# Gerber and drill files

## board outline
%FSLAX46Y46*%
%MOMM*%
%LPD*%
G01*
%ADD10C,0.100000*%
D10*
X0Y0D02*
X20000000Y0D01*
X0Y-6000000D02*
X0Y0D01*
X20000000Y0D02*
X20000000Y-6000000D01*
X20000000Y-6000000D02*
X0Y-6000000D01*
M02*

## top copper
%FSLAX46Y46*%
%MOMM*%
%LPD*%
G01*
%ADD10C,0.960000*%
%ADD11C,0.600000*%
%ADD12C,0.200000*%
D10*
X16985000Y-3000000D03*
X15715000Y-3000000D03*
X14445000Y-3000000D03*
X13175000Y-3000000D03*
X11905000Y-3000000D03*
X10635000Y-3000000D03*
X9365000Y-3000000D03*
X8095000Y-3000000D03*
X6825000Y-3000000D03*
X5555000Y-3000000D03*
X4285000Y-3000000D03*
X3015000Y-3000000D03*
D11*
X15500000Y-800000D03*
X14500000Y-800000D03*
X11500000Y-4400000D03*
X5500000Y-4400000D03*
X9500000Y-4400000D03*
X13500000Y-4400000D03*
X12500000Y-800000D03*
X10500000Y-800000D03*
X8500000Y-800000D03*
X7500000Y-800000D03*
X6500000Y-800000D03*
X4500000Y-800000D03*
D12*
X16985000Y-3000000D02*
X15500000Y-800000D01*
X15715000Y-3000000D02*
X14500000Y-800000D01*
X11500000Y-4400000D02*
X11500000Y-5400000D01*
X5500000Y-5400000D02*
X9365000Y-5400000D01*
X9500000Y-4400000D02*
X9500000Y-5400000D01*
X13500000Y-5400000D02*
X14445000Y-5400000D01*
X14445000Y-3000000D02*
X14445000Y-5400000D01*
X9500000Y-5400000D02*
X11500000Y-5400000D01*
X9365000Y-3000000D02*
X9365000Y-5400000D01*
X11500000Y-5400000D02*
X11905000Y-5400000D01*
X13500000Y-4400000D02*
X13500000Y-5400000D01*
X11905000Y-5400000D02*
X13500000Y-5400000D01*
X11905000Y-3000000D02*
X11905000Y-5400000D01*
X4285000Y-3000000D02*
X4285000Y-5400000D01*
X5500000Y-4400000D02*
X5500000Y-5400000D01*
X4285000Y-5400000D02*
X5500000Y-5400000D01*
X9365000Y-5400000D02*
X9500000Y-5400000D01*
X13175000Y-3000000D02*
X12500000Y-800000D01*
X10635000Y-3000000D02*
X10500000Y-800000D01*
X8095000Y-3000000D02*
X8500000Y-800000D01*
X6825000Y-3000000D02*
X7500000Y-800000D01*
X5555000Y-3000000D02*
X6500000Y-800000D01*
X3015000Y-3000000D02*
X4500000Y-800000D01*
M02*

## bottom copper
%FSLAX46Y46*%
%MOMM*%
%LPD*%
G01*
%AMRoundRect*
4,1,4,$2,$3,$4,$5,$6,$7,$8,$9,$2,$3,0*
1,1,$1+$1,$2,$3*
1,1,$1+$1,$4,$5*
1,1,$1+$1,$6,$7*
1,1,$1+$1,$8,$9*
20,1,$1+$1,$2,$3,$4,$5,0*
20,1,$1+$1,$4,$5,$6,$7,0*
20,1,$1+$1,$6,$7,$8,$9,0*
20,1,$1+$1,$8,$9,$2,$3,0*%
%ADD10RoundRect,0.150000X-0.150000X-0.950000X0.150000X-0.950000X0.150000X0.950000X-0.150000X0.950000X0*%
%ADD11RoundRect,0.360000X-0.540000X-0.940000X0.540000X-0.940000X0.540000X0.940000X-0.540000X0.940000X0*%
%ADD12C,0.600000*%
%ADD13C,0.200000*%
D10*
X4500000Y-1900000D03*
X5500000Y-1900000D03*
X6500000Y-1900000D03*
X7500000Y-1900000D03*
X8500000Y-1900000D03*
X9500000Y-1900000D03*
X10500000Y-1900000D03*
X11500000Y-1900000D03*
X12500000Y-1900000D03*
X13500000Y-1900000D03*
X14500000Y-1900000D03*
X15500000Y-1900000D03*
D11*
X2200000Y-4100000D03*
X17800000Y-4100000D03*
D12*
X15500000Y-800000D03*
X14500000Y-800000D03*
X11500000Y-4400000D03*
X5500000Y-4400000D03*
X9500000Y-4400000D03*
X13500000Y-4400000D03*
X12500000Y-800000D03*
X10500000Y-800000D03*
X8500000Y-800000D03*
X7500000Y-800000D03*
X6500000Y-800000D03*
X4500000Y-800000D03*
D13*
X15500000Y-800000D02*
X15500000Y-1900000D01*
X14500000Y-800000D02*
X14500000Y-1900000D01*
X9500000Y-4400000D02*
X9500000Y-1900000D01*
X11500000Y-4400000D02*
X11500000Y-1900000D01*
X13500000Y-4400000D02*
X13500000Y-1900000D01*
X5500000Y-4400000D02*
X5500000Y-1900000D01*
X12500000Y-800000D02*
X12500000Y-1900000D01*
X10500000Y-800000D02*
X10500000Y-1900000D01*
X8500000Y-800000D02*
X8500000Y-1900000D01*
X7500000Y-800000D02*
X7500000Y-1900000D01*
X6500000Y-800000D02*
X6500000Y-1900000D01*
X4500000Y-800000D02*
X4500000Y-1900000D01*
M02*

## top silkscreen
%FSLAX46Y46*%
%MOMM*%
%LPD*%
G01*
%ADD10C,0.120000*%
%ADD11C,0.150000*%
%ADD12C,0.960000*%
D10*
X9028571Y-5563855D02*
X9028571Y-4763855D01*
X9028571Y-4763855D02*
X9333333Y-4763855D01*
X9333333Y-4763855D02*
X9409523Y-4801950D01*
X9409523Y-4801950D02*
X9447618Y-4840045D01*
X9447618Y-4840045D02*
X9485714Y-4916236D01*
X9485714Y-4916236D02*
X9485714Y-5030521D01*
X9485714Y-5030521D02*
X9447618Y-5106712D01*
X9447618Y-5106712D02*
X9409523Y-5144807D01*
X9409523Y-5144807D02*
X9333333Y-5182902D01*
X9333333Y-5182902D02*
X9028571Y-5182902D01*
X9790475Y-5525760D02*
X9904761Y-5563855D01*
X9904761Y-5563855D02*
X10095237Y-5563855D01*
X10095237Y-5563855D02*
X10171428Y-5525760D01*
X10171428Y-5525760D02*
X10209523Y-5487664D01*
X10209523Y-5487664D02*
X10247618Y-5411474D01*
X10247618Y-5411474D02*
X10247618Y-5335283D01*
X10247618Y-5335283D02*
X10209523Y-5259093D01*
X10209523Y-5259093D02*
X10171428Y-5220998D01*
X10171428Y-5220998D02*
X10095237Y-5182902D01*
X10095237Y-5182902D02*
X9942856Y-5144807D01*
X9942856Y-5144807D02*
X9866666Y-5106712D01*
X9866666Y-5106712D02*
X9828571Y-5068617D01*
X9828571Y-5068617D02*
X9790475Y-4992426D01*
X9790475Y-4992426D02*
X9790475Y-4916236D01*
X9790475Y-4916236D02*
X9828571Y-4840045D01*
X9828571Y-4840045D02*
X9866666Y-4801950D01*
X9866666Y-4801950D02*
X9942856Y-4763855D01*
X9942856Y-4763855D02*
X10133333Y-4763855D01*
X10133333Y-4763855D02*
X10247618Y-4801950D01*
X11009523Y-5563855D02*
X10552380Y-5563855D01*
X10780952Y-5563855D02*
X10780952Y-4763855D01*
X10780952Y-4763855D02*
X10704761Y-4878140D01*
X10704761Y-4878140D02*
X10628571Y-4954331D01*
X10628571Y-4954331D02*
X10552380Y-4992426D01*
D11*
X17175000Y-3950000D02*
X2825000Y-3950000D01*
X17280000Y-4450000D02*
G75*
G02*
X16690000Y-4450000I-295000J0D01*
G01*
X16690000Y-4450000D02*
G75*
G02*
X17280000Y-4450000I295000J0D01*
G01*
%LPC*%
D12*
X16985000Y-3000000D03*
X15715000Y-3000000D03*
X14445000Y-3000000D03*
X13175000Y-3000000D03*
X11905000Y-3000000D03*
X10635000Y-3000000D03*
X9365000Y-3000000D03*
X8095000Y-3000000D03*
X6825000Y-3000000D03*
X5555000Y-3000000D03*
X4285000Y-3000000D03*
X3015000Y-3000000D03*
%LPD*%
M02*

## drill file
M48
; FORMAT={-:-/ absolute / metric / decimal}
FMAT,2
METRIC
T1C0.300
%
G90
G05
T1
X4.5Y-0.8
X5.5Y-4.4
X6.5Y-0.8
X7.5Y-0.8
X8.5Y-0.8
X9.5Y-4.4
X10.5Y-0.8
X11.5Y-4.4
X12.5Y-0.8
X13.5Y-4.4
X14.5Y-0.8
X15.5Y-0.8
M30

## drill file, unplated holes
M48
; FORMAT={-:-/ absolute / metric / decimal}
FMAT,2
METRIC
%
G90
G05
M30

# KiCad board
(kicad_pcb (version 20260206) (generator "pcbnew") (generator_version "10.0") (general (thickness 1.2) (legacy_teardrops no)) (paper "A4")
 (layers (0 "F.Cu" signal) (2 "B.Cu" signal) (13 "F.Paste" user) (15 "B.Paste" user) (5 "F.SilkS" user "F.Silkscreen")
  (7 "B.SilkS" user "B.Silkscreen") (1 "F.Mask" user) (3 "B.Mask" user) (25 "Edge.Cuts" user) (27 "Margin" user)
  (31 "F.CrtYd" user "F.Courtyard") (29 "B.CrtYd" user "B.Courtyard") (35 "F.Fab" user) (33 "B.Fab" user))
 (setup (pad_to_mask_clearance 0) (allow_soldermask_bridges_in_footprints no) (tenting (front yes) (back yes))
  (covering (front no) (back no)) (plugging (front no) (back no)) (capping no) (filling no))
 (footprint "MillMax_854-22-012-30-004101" (layer "F.Cu") (at 10 3 180)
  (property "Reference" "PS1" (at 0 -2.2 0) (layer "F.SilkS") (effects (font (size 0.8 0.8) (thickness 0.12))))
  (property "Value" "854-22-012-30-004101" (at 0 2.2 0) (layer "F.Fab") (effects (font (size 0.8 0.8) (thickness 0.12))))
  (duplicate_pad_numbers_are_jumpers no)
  (fp_line (start -7.175 -0.95) (end 7.175 -0.95) (stroke (width 0.15) (type solid)) (layer "F.SilkS"))
  (fp_circle (center -6.985 -1.45) (end -6.69 -1.45) (stroke (width 0.15) (type solid)) (fill no) (layer "F.SilkS"))
  (pad "1" smd circle (at -6.985 0) (size 0.96 0.96) (layers "F.Cu" "F.Mask" "F.Paste") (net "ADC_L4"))
  (pad "2" smd circle (at -5.715 0) (size 0.96 0.96) (layers "F.Cu" "F.Mask" "F.Paste") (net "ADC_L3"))
  (pad "3" smd circle (at -4.445 0) (size 0.96 0.96) (layers "F.Cu" "F.Mask" "F.Paste") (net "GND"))
  (pad "4" smd circle (at -3.175 0) (size 0.96 0.96) (layers "F.Cu" "F.Mask" "F.Paste") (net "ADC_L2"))
  (pad "5" smd circle (at -1.905 0) (size 0.96 0.96) (layers "F.Cu" "F.Mask" "F.Paste") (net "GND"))
  (pad "6" smd circle (at -0.635 0) (size 0.96 0.96) (layers "F.Cu" "F.Mask" "F.Paste") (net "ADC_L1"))
  (pad "7" smd circle (at 0.635 0) (size 0.96 0.96) (layers "F.Cu" "F.Mask" "F.Paste") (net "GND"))
  (pad "8" smd circle (at 1.905 0) (size 0.96 0.96) (layers "F.Cu" "F.Mask" "F.Paste") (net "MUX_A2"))
  (pad "9" smd circle (at 3.175 0) (size 0.96 0.96) (layers "F.Cu" "F.Mask" "F.Paste") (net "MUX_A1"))
  (pad "10" smd circle (at 4.445 0) (size 0.96 0.96) (layers "F.Cu" "F.Mask" "F.Paste") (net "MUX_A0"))
  (pad "11" smd circle (at 5.715 0) (size 0.96 0.96) (layers "F.Cu" "F.Mask" "F.Paste") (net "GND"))
  (pad "12" smd circle (at 6.985 0) (size 0.96 0.96) (layers "F.Cu" "F.Mask" "F.Paste") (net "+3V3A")))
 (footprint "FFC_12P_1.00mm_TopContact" (layer "B.Cu") (at 10 3)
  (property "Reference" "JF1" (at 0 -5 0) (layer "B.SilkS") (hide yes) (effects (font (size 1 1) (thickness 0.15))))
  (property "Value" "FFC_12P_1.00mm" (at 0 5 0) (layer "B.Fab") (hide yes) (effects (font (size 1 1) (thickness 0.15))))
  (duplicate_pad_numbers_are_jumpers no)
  (pad "1" smd roundrect (at -5.5 -1.1) (size 0.6 2.2) (layers "B.Cu" "B.Mask" "B.Paste") (roundrect_rratio 0.25) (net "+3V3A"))
  (pad "2" smd roundrect (at -4.5 -1.1) (size 0.6 2.2) (layers "B.Cu" "B.Mask" "B.Paste") (roundrect_rratio 0.25) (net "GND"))
  (pad "3" smd roundrect (at -3.5 -1.1) (size 0.6 2.2) (layers "B.Cu" "B.Mask" "B.Paste") (roundrect_rratio 0.25) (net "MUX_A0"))
  (pad "4" smd roundrect (at -2.5 -1.1) (size 0.6 2.2) (layers "B.Cu" "B.Mask" "B.Paste") (roundrect_rratio 0.25) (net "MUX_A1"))
  (pad "5" smd roundrect (at -1.5 -1.1) (size 0.6 2.2) (layers "B.Cu" "B.Mask" "B.Paste") (roundrect_rratio 0.25) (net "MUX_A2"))
  (pad "6" smd roundrect (at -0.5 -1.1) (size 0.6 2.2) (layers "B.Cu" "B.Mask" "B.Paste") (roundrect_rratio 0.25) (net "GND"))
  (pad "7" smd roundrect (at 0.5 -1.1) (size 0.6 2.2) (layers "B.Cu" "B.Mask" "B.Paste") (roundrect_rratio 0.25) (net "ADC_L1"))
  (pad "8" smd roundrect (at 1.5 -1.1) (size 0.6 2.2) (layers "B.Cu" "B.Mask" "B.Paste") (roundrect_rratio 0.25) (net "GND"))
  (pad "9" smd roundrect (at 2.5 -1.1) (size 0.6 2.2) (layers "B.Cu" "B.Mask" "B.Paste") (roundrect_rratio 0.25) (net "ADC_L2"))
  (pad "10" smd roundrect (at 3.5 -1.1) (size 0.6 2.2) (layers "B.Cu" "B.Mask" "B.Paste") (roundrect_rratio 0.25) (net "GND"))
  (pad "11" smd roundrect (at 4.5 -1.1) (size 0.6 2.2) (layers "B.Cu" "B.Mask" "B.Paste") (roundrect_rratio 0.25) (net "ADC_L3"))
  (pad "12" smd roundrect (at 5.5 -1.1) (size 0.6 2.2) (layers "B.Cu" "B.Mask" "B.Paste") (roundrect_rratio 0.25) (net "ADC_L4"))
  (pad "MP" smd roundrect (at -7.8 1.1) (size 1.8 2.6) (layers "B.Cu" "B.Mask" "B.Paste") (roundrect_rratio 0.2))
  (pad "MP" smd roundrect (at 7.8 1.1) (size 1.8 2.6) (layers "B.Cu" "B.Mask" "B.Paste") (roundrect_rratio 0.2)))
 (gr_line (start 0 0) (end 20 0) (stroke (width 0.1) (type solid)) (layer "Edge.Cuts"))
 (gr_line (start 0 6) (end 0 0) (stroke (width 0.1) (type solid)) (layer "Edge.Cuts"))
 (gr_line (start 20 0) (end 20 6) (stroke (width 0.1) (type solid)) (layer "Edge.Cuts"))
 (gr_line (start 20 6) (end 0 6) (stroke (width 0.1) (type solid)) (layer "Edge.Cuts"))
 (segment (start 16.985 3) (end 15.5 0.8) (width 0.2) (layer "F.Cu") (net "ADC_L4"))
 (via (at 15.5 0.8) (size 0.6) (drill 0.3) (layers "F.Cu" "B.Cu") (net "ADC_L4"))
 (segment (start 15.5 0.8) (end 15.5 1.9) (width 0.2) (layer "B.Cu") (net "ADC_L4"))
 (segment (start 15.715 3) (end 14.5 0.8) (width 0.2) (layer "F.Cu") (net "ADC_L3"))
 (via (at 14.5 0.8) (size 0.6) (drill 0.3) (layers "F.Cu" "B.Cu") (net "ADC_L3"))
 (segment (start 14.5 0.8) (end 14.5 1.9) (width 0.2) (layer "B.Cu") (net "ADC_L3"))
 (segment (start 11.5 4.4) (end 11.5 5.4) (width 0.2) (layer "F.Cu") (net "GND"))
 (segment (start 5.5 5.4) (end 9.365 5.4) (width 0.2) (layer "F.Cu") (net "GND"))
 (segment (start 9.5 4.4) (end 9.5 5.4) (width 0.2) (layer "F.Cu") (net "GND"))
 (segment (start 13.5 5.4) (end 14.445 5.4) (width 0.2) (layer "F.Cu") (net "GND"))
 (segment (start 14.445 3) (end 14.445 5.4) (width 0.2) (layer "F.Cu") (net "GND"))
 (segment (start 9.5 5.4) (end 11.5 5.4) (width 0.2) (layer "F.Cu") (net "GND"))
 (segment (start 9.365 3) (end 9.365 5.4) (width 0.2) (layer "F.Cu") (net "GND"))
 (segment (start 11.5 5.4) (end 11.905 5.4) (width 0.2) (layer "F.Cu") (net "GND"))
 (segment (start 13.5 4.4) (end 13.5 5.4) (width 0.2) (layer "F.Cu") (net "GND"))
 (segment (start 11.905 5.4) (end 13.5 5.4) (width 0.2) (layer "F.Cu") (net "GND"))
 (segment (start 11.905 3) (end 11.905 5.4) (width 0.2) (layer "F.Cu") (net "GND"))
 (segment (start 4.285 3) (end 4.285 5.4) (width 0.2) (layer "F.Cu") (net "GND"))
 (segment (start 5.5 4.4) (end 5.5 5.4) (width 0.2) (layer "F.Cu") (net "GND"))
 (segment (start 4.285 5.4) (end 5.5 5.4) (width 0.2) (layer "F.Cu") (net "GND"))
 (segment (start 9.365 5.4) (end 9.5 5.4) (width 0.2) (layer "F.Cu") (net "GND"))
 (via (at 11.5 4.4) (size 0.6) (drill 0.3) (layers "F.Cu" "B.Cu") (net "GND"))
 (via (at 5.5 4.4) (size 0.6) (drill 0.3) (layers "F.Cu" "B.Cu") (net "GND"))
 (via (at 9.5 4.4) (size 0.6) (drill 0.3) (layers "F.Cu" "B.Cu") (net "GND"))
 (via (at 13.5 4.4) (size 0.6) (drill 0.3) (layers "F.Cu" "B.Cu") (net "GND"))
 (segment (start 9.5 4.4) (end 9.5 1.9) (width 0.2) (layer "B.Cu") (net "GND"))
 (segment (start 11.5 4.4) (end 11.5 1.9) (width 0.2) (layer "B.Cu") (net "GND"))
 (segment (start 13.5 4.4) (end 13.5 1.9) (width 0.2) (layer "B.Cu") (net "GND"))
 (segment (start 5.5 4.4) (end 5.5 1.9) (width 0.2) (layer "B.Cu") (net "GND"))
 (segment (start 13.175 3) (end 12.5 0.8) (width 0.2) (layer "F.Cu") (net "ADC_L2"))
 (via (at 12.5 0.8) (size 0.6) (drill 0.3) (layers "F.Cu" "B.Cu") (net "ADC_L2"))
 (segment (start 12.5 0.8) (end 12.5 1.9) (width 0.2) (layer "B.Cu") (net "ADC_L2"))
 (segment (start 10.635 3) (end 10.5 0.8) (width 0.2) (layer "F.Cu") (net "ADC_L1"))
 (via (at 10.5 0.8) (size 0.6) (drill 0.3) (layers "F.Cu" "B.Cu") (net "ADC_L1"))
 (segment (start 10.5 0.8) (end 10.5 1.9) (width 0.2) (layer "B.Cu") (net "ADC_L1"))
 (segment (start 8.095 3) (end 8.5 0.8) (width 0.2) (layer "F.Cu") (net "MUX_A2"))
 (via (at 8.5 0.8) (size 0.6) (drill 0.3) (layers "F.Cu" "B.Cu") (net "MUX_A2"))
 (segment (start 8.5 0.8) (end 8.5 1.9) (width 0.2) (layer "B.Cu") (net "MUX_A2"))
 (segment (start 6.825 3) (end 7.5 0.8) (width 0.2) (layer "F.Cu") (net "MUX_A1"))
 (via (at 7.5 0.8) (size 0.6) (drill 0.3) (layers "F.Cu" "B.Cu") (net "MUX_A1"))
 (segment (start 7.5 0.8) (end 7.5 1.9) (width 0.2) (layer "B.Cu") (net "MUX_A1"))
 (segment (start 5.555 3) (end 6.5 0.8) (width 0.2) (layer "F.Cu") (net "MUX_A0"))
 (via (at 6.5 0.8) (size 0.6) (drill 0.3) (layers "F.Cu" "B.Cu") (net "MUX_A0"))
 (segment (start 6.5 0.8) (end 6.5 1.9) (width 0.2) (layer "B.Cu") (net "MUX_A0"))
 (segment (start 3.015 3) (end 4.5 0.8) (width 0.2) (layer "F.Cu") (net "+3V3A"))
 (via (at 4.5 0.8) (size 0.6) (drill 0.3) (layers "F.Cu" "B.Cu") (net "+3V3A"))
 (segment (start 4.5 0.8) (end 4.5 1.9) (width 0.2) (layer "B.Cu") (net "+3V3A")))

